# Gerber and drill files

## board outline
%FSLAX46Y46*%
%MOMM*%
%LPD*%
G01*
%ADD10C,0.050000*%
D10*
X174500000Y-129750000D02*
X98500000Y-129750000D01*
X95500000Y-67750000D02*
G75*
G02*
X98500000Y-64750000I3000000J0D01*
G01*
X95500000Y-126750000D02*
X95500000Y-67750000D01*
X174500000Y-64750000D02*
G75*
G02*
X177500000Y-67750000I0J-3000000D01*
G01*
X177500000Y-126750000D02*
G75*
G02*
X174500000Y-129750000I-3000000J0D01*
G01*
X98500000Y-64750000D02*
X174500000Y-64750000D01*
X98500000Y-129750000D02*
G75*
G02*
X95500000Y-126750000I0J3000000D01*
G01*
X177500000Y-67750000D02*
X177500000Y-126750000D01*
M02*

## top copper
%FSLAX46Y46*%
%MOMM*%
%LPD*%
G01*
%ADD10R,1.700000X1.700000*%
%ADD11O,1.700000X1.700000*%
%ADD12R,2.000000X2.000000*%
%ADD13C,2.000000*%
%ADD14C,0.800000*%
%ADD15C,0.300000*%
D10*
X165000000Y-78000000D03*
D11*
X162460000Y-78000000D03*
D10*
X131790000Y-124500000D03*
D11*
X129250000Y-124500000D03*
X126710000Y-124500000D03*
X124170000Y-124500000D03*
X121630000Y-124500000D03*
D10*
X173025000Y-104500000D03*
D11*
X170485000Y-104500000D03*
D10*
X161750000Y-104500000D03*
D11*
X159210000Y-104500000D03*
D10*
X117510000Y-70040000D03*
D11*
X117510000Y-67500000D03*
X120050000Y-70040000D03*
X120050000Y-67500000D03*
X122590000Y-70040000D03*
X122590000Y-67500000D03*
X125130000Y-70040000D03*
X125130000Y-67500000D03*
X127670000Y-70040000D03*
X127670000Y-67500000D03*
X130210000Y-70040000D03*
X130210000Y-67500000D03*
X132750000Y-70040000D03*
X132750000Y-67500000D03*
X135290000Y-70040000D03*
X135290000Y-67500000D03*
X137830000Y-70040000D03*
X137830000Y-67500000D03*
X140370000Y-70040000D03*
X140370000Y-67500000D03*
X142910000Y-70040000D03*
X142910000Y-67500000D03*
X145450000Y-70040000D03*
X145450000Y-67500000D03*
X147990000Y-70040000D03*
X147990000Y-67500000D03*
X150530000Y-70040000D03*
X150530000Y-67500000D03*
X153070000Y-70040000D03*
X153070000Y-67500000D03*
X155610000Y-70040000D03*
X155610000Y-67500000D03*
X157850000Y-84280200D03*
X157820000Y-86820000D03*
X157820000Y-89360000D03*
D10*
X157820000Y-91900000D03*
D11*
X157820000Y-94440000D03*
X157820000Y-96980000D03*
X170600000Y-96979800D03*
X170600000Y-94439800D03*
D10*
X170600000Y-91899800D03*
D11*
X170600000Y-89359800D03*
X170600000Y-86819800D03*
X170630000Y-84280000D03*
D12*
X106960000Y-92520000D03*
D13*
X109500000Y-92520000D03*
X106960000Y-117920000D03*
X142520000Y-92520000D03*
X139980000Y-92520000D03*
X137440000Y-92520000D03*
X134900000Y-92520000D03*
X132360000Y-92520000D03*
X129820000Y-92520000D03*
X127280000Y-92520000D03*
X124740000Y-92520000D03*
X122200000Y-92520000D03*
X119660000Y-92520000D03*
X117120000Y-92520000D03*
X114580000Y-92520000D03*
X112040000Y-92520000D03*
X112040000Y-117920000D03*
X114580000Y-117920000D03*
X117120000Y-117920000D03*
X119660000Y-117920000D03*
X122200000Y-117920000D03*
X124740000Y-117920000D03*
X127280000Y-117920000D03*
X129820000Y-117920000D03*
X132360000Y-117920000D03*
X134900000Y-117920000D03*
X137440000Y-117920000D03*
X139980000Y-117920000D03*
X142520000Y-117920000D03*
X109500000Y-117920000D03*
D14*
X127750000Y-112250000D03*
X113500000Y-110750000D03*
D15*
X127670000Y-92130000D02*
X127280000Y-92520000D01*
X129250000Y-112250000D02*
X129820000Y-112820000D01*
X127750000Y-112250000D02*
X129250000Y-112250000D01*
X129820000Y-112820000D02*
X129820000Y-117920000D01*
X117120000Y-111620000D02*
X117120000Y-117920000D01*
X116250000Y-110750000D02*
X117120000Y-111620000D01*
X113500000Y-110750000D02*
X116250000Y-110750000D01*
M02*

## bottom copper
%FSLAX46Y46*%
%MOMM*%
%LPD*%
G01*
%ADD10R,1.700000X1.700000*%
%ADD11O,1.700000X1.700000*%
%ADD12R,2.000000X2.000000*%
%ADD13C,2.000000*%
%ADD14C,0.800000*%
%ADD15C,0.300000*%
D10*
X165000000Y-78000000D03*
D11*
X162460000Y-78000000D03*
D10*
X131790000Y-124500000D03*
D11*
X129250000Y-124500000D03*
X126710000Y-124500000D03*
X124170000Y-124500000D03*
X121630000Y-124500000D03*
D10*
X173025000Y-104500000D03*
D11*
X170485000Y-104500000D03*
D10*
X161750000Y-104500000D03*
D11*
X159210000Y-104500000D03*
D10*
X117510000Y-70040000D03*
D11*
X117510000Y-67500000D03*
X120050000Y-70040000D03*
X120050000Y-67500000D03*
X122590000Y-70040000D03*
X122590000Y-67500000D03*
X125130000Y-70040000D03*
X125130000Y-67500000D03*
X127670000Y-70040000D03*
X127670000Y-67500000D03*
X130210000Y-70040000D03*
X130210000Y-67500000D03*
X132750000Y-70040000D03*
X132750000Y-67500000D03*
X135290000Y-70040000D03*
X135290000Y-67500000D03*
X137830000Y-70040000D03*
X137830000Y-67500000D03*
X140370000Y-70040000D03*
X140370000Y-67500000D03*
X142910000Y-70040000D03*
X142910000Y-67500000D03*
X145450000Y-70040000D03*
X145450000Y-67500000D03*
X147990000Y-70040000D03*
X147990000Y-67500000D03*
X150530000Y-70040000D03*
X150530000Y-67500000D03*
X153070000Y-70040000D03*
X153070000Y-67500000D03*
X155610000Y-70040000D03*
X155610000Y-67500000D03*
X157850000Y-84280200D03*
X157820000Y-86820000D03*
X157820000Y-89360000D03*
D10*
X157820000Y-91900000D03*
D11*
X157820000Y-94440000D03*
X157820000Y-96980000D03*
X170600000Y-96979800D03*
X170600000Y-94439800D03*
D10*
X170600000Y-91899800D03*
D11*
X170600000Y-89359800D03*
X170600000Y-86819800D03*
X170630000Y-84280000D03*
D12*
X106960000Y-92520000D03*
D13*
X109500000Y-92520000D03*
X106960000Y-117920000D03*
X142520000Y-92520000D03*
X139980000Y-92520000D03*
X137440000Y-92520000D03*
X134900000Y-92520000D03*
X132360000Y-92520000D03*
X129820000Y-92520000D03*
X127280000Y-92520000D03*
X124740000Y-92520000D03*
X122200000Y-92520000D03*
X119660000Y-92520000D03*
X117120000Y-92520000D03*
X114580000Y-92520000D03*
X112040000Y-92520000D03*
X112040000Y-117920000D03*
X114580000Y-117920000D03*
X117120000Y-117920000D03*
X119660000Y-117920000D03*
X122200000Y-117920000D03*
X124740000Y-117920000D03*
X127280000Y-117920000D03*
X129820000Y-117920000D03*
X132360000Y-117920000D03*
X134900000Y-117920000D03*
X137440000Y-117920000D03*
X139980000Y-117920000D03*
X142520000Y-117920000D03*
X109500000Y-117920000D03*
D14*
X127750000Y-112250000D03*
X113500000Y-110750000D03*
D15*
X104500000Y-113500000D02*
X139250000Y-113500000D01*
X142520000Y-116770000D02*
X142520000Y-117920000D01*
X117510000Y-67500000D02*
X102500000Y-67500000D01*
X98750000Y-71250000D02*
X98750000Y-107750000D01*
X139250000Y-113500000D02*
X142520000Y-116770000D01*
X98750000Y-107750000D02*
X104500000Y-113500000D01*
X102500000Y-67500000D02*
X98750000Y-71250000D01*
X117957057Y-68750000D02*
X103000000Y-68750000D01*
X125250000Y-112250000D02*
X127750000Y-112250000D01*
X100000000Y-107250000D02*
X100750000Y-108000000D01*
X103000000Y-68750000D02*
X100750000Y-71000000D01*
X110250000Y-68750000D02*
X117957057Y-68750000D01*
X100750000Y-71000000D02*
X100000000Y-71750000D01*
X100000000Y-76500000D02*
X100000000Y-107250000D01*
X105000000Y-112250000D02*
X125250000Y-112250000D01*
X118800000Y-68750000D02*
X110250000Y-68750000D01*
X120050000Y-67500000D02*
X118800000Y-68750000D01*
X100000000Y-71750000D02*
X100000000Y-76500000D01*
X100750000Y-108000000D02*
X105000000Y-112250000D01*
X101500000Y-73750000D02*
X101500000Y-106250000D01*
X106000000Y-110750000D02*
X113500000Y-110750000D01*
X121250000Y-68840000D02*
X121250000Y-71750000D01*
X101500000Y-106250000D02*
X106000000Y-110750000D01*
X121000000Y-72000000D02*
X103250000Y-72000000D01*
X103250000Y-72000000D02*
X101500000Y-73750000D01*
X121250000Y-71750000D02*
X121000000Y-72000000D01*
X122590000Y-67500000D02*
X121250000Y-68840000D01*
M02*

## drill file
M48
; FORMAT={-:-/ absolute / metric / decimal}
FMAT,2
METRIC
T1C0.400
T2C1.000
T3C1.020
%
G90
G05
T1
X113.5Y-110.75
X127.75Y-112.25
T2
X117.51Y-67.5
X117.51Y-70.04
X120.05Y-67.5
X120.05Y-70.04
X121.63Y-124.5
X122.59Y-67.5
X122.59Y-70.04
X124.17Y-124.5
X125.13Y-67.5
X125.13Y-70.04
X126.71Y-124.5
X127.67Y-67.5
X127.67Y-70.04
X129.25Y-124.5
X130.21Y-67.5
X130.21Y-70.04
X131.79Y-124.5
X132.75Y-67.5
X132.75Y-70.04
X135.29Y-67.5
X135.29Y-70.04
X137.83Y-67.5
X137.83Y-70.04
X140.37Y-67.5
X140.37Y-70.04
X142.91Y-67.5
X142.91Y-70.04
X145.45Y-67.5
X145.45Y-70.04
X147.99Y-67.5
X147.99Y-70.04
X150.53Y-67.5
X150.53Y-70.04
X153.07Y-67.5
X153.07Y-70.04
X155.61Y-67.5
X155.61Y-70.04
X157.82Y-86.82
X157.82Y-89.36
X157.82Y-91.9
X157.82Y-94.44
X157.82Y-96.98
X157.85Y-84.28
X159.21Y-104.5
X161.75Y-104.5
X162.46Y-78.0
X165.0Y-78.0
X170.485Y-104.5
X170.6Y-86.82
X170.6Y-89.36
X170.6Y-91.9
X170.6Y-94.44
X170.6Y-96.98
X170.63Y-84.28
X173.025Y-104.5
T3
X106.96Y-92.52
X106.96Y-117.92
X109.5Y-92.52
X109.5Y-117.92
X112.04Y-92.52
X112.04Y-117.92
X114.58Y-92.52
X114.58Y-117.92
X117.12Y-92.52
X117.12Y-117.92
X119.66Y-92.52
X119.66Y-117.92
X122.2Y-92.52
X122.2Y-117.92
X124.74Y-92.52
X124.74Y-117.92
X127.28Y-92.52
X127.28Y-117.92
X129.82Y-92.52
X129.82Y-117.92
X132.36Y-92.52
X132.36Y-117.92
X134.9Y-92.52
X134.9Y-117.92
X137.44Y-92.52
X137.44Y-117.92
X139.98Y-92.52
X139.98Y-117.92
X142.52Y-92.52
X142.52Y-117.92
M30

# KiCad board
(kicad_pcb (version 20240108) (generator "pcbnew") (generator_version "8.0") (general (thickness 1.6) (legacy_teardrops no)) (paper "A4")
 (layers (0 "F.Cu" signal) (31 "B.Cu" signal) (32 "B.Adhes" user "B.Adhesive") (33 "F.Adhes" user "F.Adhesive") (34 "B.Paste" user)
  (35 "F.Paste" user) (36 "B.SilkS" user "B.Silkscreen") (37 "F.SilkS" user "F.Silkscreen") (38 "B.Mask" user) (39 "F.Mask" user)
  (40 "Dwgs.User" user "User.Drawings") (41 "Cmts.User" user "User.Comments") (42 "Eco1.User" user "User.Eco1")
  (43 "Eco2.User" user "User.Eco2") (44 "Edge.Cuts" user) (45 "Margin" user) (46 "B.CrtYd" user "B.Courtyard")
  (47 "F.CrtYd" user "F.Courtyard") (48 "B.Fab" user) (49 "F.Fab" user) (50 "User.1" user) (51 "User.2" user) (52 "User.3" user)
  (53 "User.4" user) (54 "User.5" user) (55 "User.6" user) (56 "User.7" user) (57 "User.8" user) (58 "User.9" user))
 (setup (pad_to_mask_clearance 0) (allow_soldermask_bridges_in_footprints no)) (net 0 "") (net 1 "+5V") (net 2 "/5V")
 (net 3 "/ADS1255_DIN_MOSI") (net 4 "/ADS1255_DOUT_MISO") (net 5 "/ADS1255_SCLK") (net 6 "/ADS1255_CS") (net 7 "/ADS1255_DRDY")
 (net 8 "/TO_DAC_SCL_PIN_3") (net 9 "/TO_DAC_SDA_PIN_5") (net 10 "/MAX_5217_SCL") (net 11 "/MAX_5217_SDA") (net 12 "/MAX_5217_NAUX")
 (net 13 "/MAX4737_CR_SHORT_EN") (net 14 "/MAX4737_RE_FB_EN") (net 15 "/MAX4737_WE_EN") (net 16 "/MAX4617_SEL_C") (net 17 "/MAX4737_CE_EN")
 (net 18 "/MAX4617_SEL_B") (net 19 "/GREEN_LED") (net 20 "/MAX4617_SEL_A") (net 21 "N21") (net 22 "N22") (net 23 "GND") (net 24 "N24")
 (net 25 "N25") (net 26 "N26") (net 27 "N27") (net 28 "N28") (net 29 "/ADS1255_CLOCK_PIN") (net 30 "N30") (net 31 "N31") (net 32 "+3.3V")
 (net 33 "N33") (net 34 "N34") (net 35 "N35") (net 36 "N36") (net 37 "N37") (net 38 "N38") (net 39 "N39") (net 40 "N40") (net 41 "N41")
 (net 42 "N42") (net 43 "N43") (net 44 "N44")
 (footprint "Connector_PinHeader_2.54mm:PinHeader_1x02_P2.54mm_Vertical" (layer "F.Cu") (at 165 78 -90)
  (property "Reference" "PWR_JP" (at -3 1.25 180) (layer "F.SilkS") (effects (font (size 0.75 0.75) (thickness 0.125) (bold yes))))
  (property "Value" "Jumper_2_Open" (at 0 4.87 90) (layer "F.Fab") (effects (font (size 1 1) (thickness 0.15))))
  (pad "1" thru_hole rect (at 0 0 270) (size 1.7 1.7) (drill 1) (layers "*.Cu" "*.Mask") (remove_unused_layers no) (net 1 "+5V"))
  (pad "2" thru_hole oval (at 0 2.54 270) (size 1.7 1.7) (drill 1) (layers "*.Cu" "*.Mask") (remove_unused_layers no) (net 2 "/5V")))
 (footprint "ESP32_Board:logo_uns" (layer "F.Cu") (at 164.5 121.5)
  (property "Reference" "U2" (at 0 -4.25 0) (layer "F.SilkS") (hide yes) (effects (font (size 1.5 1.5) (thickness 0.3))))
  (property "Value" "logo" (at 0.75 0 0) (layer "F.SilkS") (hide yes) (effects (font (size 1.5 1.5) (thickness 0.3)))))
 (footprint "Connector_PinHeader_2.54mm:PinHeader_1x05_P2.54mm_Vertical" (layer "F.Cu") (at 131.79 124.5 -90)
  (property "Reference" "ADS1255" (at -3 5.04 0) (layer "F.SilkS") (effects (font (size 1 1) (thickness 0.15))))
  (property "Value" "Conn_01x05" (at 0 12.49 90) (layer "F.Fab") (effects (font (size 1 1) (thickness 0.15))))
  (pad "1" thru_hole rect (at 0 0 270) (size 1.7 1.7) (drill 1) (layers "*.Cu" "*.Mask") (remove_unused_layers no)
   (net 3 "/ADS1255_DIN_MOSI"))
  (pad "2" thru_hole oval (at 0 2.54 270) (size 1.7 1.7) (drill 1) (layers "*.Cu" "*.Mask") (remove_unused_layers no)
   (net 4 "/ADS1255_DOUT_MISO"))
  (pad "3" thru_hole oval (at 0 5.08 270) (size 1.7 1.7) (drill 1) (layers "*.Cu" "*.Mask") (remove_unused_layers no)
   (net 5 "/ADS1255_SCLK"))
  (pad "4" thru_hole oval (at 0 7.62 270) (size 1.7 1.7) (drill 1) (layers "*.Cu" "*.Mask") (remove_unused_layers no) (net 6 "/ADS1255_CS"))
  (pad "5" thru_hole oval (at 0 10.16 270) (size 1.7 1.7) (drill 1) (layers "*.Cu" "*.Mask") (remove_unused_layers no)
   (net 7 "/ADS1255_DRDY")))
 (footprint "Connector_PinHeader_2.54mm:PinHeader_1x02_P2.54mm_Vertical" (layer "F.Cu") (at 173.025 104.5 -90)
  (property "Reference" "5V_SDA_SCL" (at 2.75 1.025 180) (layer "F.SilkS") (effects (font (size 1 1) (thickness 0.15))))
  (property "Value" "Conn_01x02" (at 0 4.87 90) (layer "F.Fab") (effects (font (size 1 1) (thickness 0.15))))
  (pad "1" thru_hole rect (at 0 0 270) (size 1.7 1.7) (drill 1) (layers "*.Cu" "*.Mask") (remove_unused_layers no)
   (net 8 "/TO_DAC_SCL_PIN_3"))
  (pad "2" thru_hole oval (at 0 2.54 270) (size 1.7 1.7) (drill 1) (layers "*.Cu" "*.Mask") (remove_unused_layers no)
   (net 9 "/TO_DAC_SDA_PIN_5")))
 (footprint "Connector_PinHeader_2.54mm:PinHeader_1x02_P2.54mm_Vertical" (layer "F.Cu") (at 161.75 104.5 -90)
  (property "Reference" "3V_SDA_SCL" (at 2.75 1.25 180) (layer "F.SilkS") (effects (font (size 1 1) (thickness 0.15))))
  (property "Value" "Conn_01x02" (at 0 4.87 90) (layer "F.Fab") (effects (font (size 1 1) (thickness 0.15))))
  (pad "1" thru_hole rect (at 0 0 270) (size 1.7 1.7) (drill 1) (layers "*.Cu" "*.Mask") (remove_unused_layers no) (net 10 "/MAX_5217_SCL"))
  (pad "2" thru_hole oval (at 0 2.54 270) (size 1.7 1.7) (drill 1) (layers "*.Cu" "*.Mask") (remove_unused_layers no)
   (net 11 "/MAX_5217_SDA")))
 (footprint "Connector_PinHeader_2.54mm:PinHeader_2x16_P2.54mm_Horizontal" (layer "F.Cu") (at 117.51 70.04 90)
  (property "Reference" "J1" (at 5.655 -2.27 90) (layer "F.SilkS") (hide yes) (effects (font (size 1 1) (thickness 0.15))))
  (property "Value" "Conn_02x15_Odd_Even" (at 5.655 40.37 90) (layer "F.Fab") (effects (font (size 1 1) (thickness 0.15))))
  (pad "1" thru_hole rect (at 0 0 90) (size 1.7 1.7) (drill 1) (layers "*.Cu" "*.Mask") (remove_unused_layers no) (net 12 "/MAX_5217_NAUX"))
  (pad "2" thru_hole oval (at 2.54 0 90) (size 1.7 1.7) (drill 1) (layers "*.Cu" "*.Mask") (remove_unused_layers no)
   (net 3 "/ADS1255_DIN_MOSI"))
  (pad "3" thru_hole oval (at 0 2.54 90) (size 1.7 1.7) (drill 1) (layers "*.Cu" "*.Mask") (remove_unused_layers no)
   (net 8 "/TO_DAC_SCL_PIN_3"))
  (pad "4" thru_hole oval (at 2.54 2.54 90) (size 1.7 1.7) (drill 1) (layers "*.Cu" "*.Mask") (remove_unused_layers no)
   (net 4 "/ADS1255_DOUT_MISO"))
  (pad "5" thru_hole oval (at 0 5.08 90) (size 1.7 1.7) (drill 1) (layers "*.Cu" "*.Mask") (remove_unused_layers no)
   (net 9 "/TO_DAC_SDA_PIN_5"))
  (pad "6" thru_hole oval (at 2.54 5.08 90) (size 1.7 1.7) (drill 1) (layers "*.Cu" "*.Mask") (remove_unused_layers no)
   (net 7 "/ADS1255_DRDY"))
  (pad "7" thru_hole oval (at 0 7.62 90) (size 1.7 1.7) (drill 1) (layers "*.Cu" "*.Mask") (remove_unused_layers no)
   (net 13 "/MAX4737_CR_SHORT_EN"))
  (pad "8" thru_hole oval (at 2.54 7.62 90) (size 1.7 1.7) (drill 1) (layers "*.Cu" "*.Mask") (remove_unused_layers no)
   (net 6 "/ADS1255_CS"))
  (pad "9" thru_hole oval (at 0 10.16 90) (size 1.7 1.7) (drill 1) (layers "*.Cu" "*.Mask") (remove_unused_layers no)
   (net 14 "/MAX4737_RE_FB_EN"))
  (pad "10" thru_hole oval (at 2.54 10.16 90) (size 1.7 1.7) (drill 1) (layers "*.Cu" "*.Mask") (remove_unused_layers no)
   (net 5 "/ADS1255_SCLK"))
  (pad "11" thru_hole oval (at 0 12.7 90) (size 1.7 1.7) (drill 1) (layers "*.Cu" "*.Mask") (remove_unused_layers no)
   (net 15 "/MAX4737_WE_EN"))
  (pad "12" thru_hole oval (at 2.54 12.7 90) (size 1.7 1.7) (drill 1) (layers "*.Cu" "*.Mask") (remove_unused_layers no)
   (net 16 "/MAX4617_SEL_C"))
  (pad "13" thru_hole oval (at 0 15.24 90) (size 1.7 1.7) (drill 1) (layers "*.Cu" "*.Mask") (remove_unused_layers no)
   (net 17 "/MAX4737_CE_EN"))
  (pad "14" thru_hole oval (at 2.54 15.24 90) (size 1.7 1.7) (drill 1) (layers "*.Cu" "*.Mask") (remove_unused_layers no)
   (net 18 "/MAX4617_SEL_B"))
  (pad "15" thru_hole oval (at 0 17.78 90) (size 1.7 1.7) (drill 1) (layers "*.Cu" "*.Mask") (remove_unused_layers no) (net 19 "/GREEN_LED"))
  (pad "16" thru_hole oval (at 2.54 17.78 90) (size 1.7 1.7) (drill 1) (layers "*.Cu" "*.Mask") (remove_unused_layers no)
   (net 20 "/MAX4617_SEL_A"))
  (pad "17" thru_hole oval (at 0 20.32 90) (size 1.7 1.7) (drill 1) (layers "*.Cu" "*.Mask") (remove_unused_layers no) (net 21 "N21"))
  (pad "18" thru_hole oval (at 2.54 20.32 90) (size 1.7 1.7) (drill 1) (layers "*.Cu" "*.Mask") (remove_unused_layers no) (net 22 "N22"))
  (pad "19" thru_hole oval (at 0 22.86 90) (size 1.7 1.7) (drill 1) (layers "*.Cu" "*.Mask") (remove_unused_layers no) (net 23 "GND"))
  (pad "20" thru_hole oval (at 2.54 22.86 90) (size 1.7 1.7) (drill 1) (layers "*.Cu" "*.Mask") (remove_unused_layers no) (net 23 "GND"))
  (pad "21" thru_hole oval (at 0 25.4 90) (size 1.7 1.7) (drill 1) (layers "*.Cu" "*.Mask") (remove_unused_layers no) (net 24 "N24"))
  (pad "22" thru_hole oval (at 2.54 25.4 90) (size 1.7 1.7) (drill 1) (layers "*.Cu" "*.Mask") (remove_unused_layers no) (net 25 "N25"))
  (pad "23" thru_hole oval (at 0 27.94 90) (size 1.7 1.7) (drill 1) (layers "*.Cu" "*.Mask") (remove_unused_layers no) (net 2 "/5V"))
  (pad "24" thru_hole oval (at 2.54 27.94 90) (size 1.7 1.7) (drill 1) (layers "*.Cu" "*.Mask") (remove_unused_layers no) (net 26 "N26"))
  (pad "25" thru_hole oval (at 0 30.48 90) (size 1.7 1.7) (drill 1) (layers "*.Cu" "*.Mask") (remove_unused_layers no) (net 23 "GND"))
  (pad "26" thru_hole oval (at 2.54 30.48 90) (size 1.7 1.7) (drill 1) (layers "*.Cu" "*.Mask") (remove_unused_layers no) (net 23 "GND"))
  (pad "27" thru_hole oval (at 0 33.02 90) (size 1.7 1.7) (drill 1) (layers "*.Cu" "*.Mask") (remove_unused_layers no) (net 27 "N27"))
  (pad "28" thru_hole oval (at 2.54 33.02 90) (size 1.7 1.7) (drill 1) (layers "*.Cu" "*.Mask") (remove_unused_layers no) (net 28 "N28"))
  (pad "29" thru_hole oval (at 0 35.56 90) (size 1.7 1.7) (drill 1) (layers "*.Cu" "*.Mask") (remove_unused_layers no)
   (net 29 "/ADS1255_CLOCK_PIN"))
  (pad "30" thru_hole oval (at 2.54 35.56 90) (size 1.7 1.7) (drill 1) (layers "*.Cu" "*.Mask") (remove_unused_layers no) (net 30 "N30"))
  (pad "31" thru_hole oval (at 0 38.1 90) (size 1.7 1.7) (drill 1) (layers "*.Cu" "*.Mask") (remove_unused_layers no))
  (pad "32" thru_hole oval (at 2.54 38.1 90) (size 1.7 1.7) (drill 1) (layers "*.Cu" "*.Mask") (remove_unused_layers no)))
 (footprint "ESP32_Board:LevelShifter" (layer "F.Cu") (at 164 90.75)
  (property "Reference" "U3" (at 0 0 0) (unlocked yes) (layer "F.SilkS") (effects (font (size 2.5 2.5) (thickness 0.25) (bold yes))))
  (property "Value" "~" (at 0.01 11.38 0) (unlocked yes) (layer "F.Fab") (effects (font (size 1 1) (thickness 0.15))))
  (pad "1" thru_hole oval (at -6.15 -6.4698) (size 1.7 1.7) (drill 1) (layers "*.Cu" "*.Mask") (remove_unused_layers no)
   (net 10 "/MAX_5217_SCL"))
  (pad "2" thru_hole oval (at -6.18 -3.93) (size 1.7 1.7) (drill 1) (layers "*.Cu" "*.Mask") (remove_unused_layers no) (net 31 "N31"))
  (pad "3" thru_hole oval (at -6.18 -1.39) (size 1.7 1.7) (drill 1) (layers "*.Cu" "*.Mask") (remove_unused_layers no) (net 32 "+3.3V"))
  (pad "4" thru_hole rect (at -6.18 1.15) (size 1.7 1.7) (drill 1) (layers "*.Cu" "*.Mask") (remove_unused_layers no) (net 23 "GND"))
  (pad "5" thru_hole oval (at -6.18 3.69) (size 1.7 1.7) (drill 1) (layers "*.Cu" "*.Mask") (remove_unused_layers no) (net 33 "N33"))
  (pad "6" thru_hole oval (at -6.18 6.23) (size 1.7 1.7) (drill 1) (layers "*.Cu" "*.Mask") (remove_unused_layers no)
   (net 11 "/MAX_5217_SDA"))
  (pad "7" thru_hole oval (at 6.6 6.2298) (size 1.7 1.7) (drill 1) (layers "*.Cu" "*.Mask") (remove_unused_layers no)
   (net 9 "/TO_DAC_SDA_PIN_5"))
  (pad "8" thru_hole oval (at 6.6 3.6898) (size 1.7 1.7) (drill 1) (layers "*.Cu" "*.Mask") (remove_unused_layers no) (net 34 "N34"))
  (pad "9" thru_hole rect (at 6.6 1.1498) (size 1.7 1.7) (drill 1) (layers "*.Cu" "*.Mask") (remove_unused_layers no) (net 23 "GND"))
  (pad "10" thru_hole oval (at 6.6 -1.3902) (size 1.7 1.7) (drill 1) (layers "*.Cu" "*.Mask") (remove_unused_layers no) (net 1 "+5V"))
  (pad "11" thru_hole oval (at 6.6 -3.9302) (size 1.7 1.7) (drill 1) (layers "*.Cu" "*.Mask") (remove_unused_layers no) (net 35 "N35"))
  (pad "12" thru_hole oval (at 6.63 -6.47) (size 1.7 1.7) (drill 1) (layers "*.Cu" "*.Mask") (remove_unused_layers no)
   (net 8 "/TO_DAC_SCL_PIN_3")))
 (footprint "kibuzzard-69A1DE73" (layer "F.Cu") (at 127 127.5)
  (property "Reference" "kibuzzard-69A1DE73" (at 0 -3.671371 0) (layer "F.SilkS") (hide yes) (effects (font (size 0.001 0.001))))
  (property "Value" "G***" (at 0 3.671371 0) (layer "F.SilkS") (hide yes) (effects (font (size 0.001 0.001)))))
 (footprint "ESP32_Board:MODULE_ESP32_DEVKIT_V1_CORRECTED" (layer "F.Cu") (at 122.75 105.25 -90)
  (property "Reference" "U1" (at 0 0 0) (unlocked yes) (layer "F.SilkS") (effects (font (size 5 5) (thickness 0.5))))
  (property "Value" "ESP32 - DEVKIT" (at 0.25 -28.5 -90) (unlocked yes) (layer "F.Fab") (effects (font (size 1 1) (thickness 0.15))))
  (pad "0" thru_hole rect (at -12.73 15.79 90) (size 2 2) (drill 1.02) (layers "*.Cu" "*.Mask") (remove_unused_layers no) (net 1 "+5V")
   (solder_mask_margin 0.102))
  (pad "1" thru_hole circle (at -12.73 13.25 90) (size 2 2) (drill 1.02) (layers "*.Cu" "*.Mask") (remove_unused_layers no) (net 23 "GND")
   (solder_mask_margin 0.102))
  (pad "2" thru_hole circle (at 12.67 15.79 90) (size 2 2) (drill 1.02) (layers "*.Cu" "*.Mask") (remove_unused_layers no) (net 32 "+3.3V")
   (solder_mask_margin 0.102))
  (pad "3" thru_hole circle (at -12.73 -19.77 90) (size 2 2) (drill 1.02) (layers "*.Cu" "*.Mask") (remove_unused_layers no) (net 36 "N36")
   (solder_mask_margin 0.102))
  (pad "4" thru_hole circle (at -12.73 -17.23 90) (size 2 2) (drill 1.02) (layers "*.Cu" "*.Mask") (remove_unused_layers no) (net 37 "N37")
   (solder_mask_margin 0.102))
  (pad "5" thru_hole circle (at -12.73 -14.69 90) (size 2 2) (drill 1.02) (layers "*.Cu" "*.Mask") (remove_unused_layers no) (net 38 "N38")
   (solder_mask_margin 0.102))
  (pad "6" thru_hole circle (at -12.73 -12.15 90) (size 2 2) (drill 1.02) (layers "*.Cu" "*.Mask") (remove_unused_layers no) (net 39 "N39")
   (solder_mask_margin 0.102))
  (pad "7" thru_hole circle (at -12.73 -9.61 90) (size 2 2) (drill 1.02) (layers "*.Cu" "*.Mask") (remove_unused_layers no) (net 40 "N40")
   (solder_mask_margin 0.102))
  (pad "8" thru_hole circle (at -12.73 -7.07 90) (size 2 2) (drill 1.02) (layers "*.Cu" "*.Mask") (remove_unused_layers no)
   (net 12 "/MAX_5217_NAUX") (solder_mask_margin 0.102))
  (pad "9" thru_hole circle (at -12.73 -4.53 90) (size 2 2) (drill 1.02) (layers "*.Cu" "*.Mask") (remove_unused_layers no)
   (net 14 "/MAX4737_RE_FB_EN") (solder_mask_margin 0.102))
  (pad "10" thru_hole circle (at -12.73 -1.99 90) (size 2 2) (drill 1.02) (layers "*.Cu" "*.Mask") (remove_unused_layers no)
   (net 16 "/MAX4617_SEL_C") (solder_mask_margin 0.102))
  (pad "11" thru_hole circle (at -12.73 0.55 90) (size 2 2) (drill 1.02) (layers "*.Cu" "*.Mask") (remove_unused_layers no)
   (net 18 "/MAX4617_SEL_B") (solder_mask_margin 0.102))
  (pad "12" thru_hole circle (at -12.73 3.09 90) (size 2 2) (drill 1.02) (layers "*.Cu" "*.Mask") (remove_unused_layers no)
   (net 20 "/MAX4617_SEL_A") (solder_mask_margin 0.102))
  (pad "13" thru_hole circle (at -12.73 5.63 90) (size 2 2) (drill 1.02) (layers "*.Cu" "*.Mask") (remove_unused_layers no)
   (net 13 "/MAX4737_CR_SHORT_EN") (solder_mask_margin 0.102))
  (pad "14" thru_hole circle (at -12.73 8.17 90) (size 2 2) (drill 1.02) (layers "*.Cu" "*.Mask") (remove_unused_layers no) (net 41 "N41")
   (solder_mask_margin 0.102))
  (pad "16" thru_hole circle (at -12.73 10.71 90) (size 2 2) (drill 1.02) (layers "*.Cu" "*.Mask") (remove_unused_layers no)
   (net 15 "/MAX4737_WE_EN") (solder_mask_margin 0.102))
  (pad "23" thru_hole circle (at 12.67 10.71 90) (size 2 2) (drill 1.02) (layers "*.Cu" "*.Mask") (remove_unused_layers no)
   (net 17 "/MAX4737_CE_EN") (solder_mask_margin 0.102))
  (pad "24" thru_hole circle (at 12.67 8.17 90) (size 2 2) (drill 1.02) (layers "*.Cu" "*.Mask") (remove_unused_layers no)
   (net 19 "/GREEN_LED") (solder_mask_margin 0.102))
  (pad "26" thru_hole circle (at 12.67 5.63 90) (size 2 2) (drill 1.02) (layers "*.Cu" "*.Mask") (remove_unused_layers no)
   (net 7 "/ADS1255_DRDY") (solder_mask_margin 0.102))
  (pad "27" thru_hole circle (at 12.67 3.09 90) (size 2 2) (drill 1.02) (layers "*.Cu" "*.Mask") (remove_unused_layers no)
   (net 29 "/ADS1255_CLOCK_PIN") (solder_mask_margin 0.102))
  (pad "28" thru_hole circle (at 12.67 0.55 90) (size 2 2) (drill 1.02) (layers "*.Cu" "*.Mask") (remove_unused_layers no) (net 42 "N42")
   (solder_mask_margin 0.102))
  (pad "29" thru_hole circle (at 12.67 -1.99 90) (size 2 2) (drill 1.02) (layers "*.Cu" "*.Mask") (remove_unused_layers no)
   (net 6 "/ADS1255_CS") (solder_mask_margin 0.102))
  (pad "30" thru_hole circle (at 12.67 -4.53 90) (size 2 2) (drill 1.02) (layers "*.Cu" "*.Mask") (remove_unused_layers no)
   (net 5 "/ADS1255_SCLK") (solder_mask_margin 0.102))
  (pad "31" thru_hole circle (at 12.67 -7.07 90) (size 2 2) (drill 1.02) (layers "*.Cu" "*.Mask") (remove_unused_layers no)
   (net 4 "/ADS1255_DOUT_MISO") (solder_mask_margin 0.102))
  (pad "33" thru_hole circle (at 12.67 -9.61 90) (size 2 2) (drill 1.02) (layers "*.Cu" "*.Mask") (remove_unused_layers no)
   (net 11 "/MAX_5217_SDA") (solder_mask_margin 0.102))
  (pad "34" thru_hole circle (at 12.67 -12.15 90) (size 2 2) (drill 1.02) (layers "*.Cu" "*.Mask") (remove_unused_layers no) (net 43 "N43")
   (solder_mask_margin 0.102))
  (pad "35" thru_hole circle (at 12.67 -14.69 90) (size 2 2) (drill 1.02) (layers "*.Cu" "*.Mask") (remove_unused_layers no) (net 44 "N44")
   (solder_mask_margin 0.102))
  (pad "36" thru_hole circle (at 12.67 -17.23 90) (size 2 2) (drill 1.02) (layers "*.Cu" "*.Mask") (remove_unused_layers no)
   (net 10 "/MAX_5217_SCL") (solder_mask_margin 0.102))
  (pad "37" thru_hole circle (at 12.67 -19.77 90) (size 2 2) (drill 1.02) (layers "*.Cu" "*.Mask") (remove_unused_layers no)
   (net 3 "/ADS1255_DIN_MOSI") (solder_mask_margin 0.102))
  (pad "38" thru_hole circle (at 12.67 13.25 90) (size 2 2) (drill 1.02) (layers "*.Cu" "*.Mask") (remove_unused_layers no) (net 23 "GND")
   (solder_mask_margin 0.102))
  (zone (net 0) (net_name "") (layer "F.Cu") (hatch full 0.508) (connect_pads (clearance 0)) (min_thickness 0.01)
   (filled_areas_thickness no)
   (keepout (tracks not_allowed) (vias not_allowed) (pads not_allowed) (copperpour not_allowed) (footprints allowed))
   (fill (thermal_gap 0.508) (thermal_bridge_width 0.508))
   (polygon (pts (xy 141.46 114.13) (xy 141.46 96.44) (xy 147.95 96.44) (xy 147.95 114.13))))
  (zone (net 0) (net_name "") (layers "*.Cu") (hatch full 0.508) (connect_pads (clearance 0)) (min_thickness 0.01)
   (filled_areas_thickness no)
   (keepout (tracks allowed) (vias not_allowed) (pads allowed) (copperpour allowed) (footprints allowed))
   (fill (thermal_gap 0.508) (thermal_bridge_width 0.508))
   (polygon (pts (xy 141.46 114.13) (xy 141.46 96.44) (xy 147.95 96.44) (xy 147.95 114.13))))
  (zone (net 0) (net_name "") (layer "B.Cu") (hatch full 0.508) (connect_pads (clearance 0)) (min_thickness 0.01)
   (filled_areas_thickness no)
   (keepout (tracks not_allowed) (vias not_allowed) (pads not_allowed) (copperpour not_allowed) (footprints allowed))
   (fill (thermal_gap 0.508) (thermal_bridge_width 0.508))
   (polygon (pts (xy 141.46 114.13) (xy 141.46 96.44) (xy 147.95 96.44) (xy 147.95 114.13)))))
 (gr_line (start 174.5 129.75) (end 98.5 129.75) (stroke (width 0.05) (type default)) (layer "Edge.Cuts"))
 (gr_arc (start 95.5 67.75) (mid 96.37868 65.62868) (end 98.5 64.75) (stroke (width 0.05) (type default)) (layer "Edge.Cuts"))
 (gr_line (start 95.5 126.75) (end 95.5 67.75) (stroke (width 0.05) (type default)) (layer "Edge.Cuts"))
 (gr_arc (start 174.5 64.75) (mid 176.62132 65.62868) (end 177.5 67.75) (stroke (width 0.05) (type default)) (layer "Edge.Cuts"))
 (gr_arc (start 177.5 126.75) (mid 176.62132 128.87132) (end 174.5 129.75) (stroke (width 0.05) (type default)) (layer "Edge.Cuts"))
 (gr_line (start 98.5 64.75) (end 174.5 64.75) (stroke (width 0.05) (type default)) (layer "Edge.Cuts"))
 (gr_arc (start 98.5 129.75) (mid 96.37868 128.87132) (end 95.5 126.75) (stroke (width 0.05) (type default)) (layer "Edge.Cuts"))
 (gr_line (start 177.5 67.75) (end 177.5 126.75) (stroke (width 0.05) (type default)) (layer "Edge.Cuts"))
 (segment (start 127.67 92.13) (end 127.28 92.52) (width 0.3) (layer "F.Cu") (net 14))
 (segment (start 104.5 113.5) (end 139.25 113.5) (width 0.3) (layer "B.Cu") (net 3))
 (segment (start 142.52 116.77) (end 142.52 117.92) (width 0.3) (layer "B.Cu") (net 3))
 (segment (start 117.51 67.5) (end 102.5 67.5) (width 0.3) (layer "B.Cu") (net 3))
 (segment (start 98.75 71.25) (end 98.75 107.75) (width 0.3) (layer "B.Cu") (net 3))
 (segment (start 139.25 113.5) (end 142.52 116.77) (width 0.3) (layer "B.Cu") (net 3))
 (segment (start 98.75 107.75) (end 104.5 113.5) (width 0.3) (layer "B.Cu") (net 3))
 (segment (start 102.5 67.5) (end 98.75 71.25) (width 0.3) (layer "B.Cu") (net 3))
 (segment (start 129.25 112.25) (end 129.82 112.82) (width 0.3) (layer "F.Cu") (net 4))
 (segment (start 127.75 112.25) (end 129.25 112.25) (width 0.3) (layer "F.Cu") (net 4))
 (segment (start 129.82 112.82) (end 129.82 117.92) (width 0.3) (layer "F.Cu") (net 4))
 (via (at 127.75 112.25) (size 0.8) (drill 0.4) (layers "F.Cu" "B.Cu") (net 4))
 (segment (start 117.957057 68.75) (end 103 68.75) (width 0.3) (layer "B.Cu") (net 4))
 (segment (start 125.25 112.25) (end 127.75 112.25) (width 0.3) (layer "B.Cu") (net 4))
 (segment (start 100 107.25) (end 100.75 108) (width 0.3) (layer "B.Cu") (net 4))
 (segment (start 103 68.75) (end 100.75 71) (width 0.3) (layer "B.Cu") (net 4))
 (segment (start 110.25 68.75) (end 117.957057 68.75) (width 0.3) (layer "B.Cu") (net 4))
 (segment (start 100.75 71) (end 100 71.75) (width 0.3) (layer "B.Cu") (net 4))
 (segment (start 100 76.5) (end 100 107.25) (width 0.3) (layer "B.Cu") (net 4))
 (segment (start 105 112.25) (end 125.25 112.25) (width 0.3) (layer "B.Cu") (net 4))
 (segment (start 118.8 68.75) (end 110.25 68.75) (width 0.3) (layer "B.Cu") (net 4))
 (segment (start 120.05 67.5) (end 118.8 68.75) (width 0.3) (layer "B.Cu") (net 4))
 (segment (start 100 71.75) (end 100 76.5) (width 0.3) (layer "B.Cu") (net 4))
 (segment (start 100.75 108) (end 105 112.25) (width 0.3) (layer "B.Cu") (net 4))
 (segment (start 117.12 111.62) (end 117.12 117.92) (width 0.3) (layer "F.Cu") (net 7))
 (segment (start 116.25 110.75) (end 117.12 111.62) (width 0.3) (layer "F.Cu") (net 7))
 (segment (start 113.5 110.75) (end 116.25 110.75) (width 0.3) (layer "F.Cu") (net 7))
 (via (at 113.5 110.75) (size 0.8) (drill 0.4) (layers "F.Cu" "B.Cu") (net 7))
 (segment (start 101.5 73.75) (end 101.5 106.25) (width 0.3) (layer "B.Cu") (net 7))
 (segment (start 106 110.75) (end 113.5 110.75) (width 0.3) (layer "B.Cu") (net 7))
 (segment (start 121.25 68.84) (end 121.25 71.75) (width 0.3) (layer "B.Cu") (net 7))
 (segment (start 101.5 106.25) (end 106 110.75) (width 0.3) (layer "B.Cu") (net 7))
 (segment (start 121 72) (end 103.25 72) (width 0.3) (layer "B.Cu") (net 7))
 (segment (start 103.25 72) (end 101.5 73.75) (width 0.3) (layer "B.Cu") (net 7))
 (segment (start 121.25 71.75) (end 121 72) (width 0.3) (layer "B.Cu") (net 7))
 (segment (start 122.59 67.5) (end 121.25 68.84) (width 0.3) (layer "B.Cu") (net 7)))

